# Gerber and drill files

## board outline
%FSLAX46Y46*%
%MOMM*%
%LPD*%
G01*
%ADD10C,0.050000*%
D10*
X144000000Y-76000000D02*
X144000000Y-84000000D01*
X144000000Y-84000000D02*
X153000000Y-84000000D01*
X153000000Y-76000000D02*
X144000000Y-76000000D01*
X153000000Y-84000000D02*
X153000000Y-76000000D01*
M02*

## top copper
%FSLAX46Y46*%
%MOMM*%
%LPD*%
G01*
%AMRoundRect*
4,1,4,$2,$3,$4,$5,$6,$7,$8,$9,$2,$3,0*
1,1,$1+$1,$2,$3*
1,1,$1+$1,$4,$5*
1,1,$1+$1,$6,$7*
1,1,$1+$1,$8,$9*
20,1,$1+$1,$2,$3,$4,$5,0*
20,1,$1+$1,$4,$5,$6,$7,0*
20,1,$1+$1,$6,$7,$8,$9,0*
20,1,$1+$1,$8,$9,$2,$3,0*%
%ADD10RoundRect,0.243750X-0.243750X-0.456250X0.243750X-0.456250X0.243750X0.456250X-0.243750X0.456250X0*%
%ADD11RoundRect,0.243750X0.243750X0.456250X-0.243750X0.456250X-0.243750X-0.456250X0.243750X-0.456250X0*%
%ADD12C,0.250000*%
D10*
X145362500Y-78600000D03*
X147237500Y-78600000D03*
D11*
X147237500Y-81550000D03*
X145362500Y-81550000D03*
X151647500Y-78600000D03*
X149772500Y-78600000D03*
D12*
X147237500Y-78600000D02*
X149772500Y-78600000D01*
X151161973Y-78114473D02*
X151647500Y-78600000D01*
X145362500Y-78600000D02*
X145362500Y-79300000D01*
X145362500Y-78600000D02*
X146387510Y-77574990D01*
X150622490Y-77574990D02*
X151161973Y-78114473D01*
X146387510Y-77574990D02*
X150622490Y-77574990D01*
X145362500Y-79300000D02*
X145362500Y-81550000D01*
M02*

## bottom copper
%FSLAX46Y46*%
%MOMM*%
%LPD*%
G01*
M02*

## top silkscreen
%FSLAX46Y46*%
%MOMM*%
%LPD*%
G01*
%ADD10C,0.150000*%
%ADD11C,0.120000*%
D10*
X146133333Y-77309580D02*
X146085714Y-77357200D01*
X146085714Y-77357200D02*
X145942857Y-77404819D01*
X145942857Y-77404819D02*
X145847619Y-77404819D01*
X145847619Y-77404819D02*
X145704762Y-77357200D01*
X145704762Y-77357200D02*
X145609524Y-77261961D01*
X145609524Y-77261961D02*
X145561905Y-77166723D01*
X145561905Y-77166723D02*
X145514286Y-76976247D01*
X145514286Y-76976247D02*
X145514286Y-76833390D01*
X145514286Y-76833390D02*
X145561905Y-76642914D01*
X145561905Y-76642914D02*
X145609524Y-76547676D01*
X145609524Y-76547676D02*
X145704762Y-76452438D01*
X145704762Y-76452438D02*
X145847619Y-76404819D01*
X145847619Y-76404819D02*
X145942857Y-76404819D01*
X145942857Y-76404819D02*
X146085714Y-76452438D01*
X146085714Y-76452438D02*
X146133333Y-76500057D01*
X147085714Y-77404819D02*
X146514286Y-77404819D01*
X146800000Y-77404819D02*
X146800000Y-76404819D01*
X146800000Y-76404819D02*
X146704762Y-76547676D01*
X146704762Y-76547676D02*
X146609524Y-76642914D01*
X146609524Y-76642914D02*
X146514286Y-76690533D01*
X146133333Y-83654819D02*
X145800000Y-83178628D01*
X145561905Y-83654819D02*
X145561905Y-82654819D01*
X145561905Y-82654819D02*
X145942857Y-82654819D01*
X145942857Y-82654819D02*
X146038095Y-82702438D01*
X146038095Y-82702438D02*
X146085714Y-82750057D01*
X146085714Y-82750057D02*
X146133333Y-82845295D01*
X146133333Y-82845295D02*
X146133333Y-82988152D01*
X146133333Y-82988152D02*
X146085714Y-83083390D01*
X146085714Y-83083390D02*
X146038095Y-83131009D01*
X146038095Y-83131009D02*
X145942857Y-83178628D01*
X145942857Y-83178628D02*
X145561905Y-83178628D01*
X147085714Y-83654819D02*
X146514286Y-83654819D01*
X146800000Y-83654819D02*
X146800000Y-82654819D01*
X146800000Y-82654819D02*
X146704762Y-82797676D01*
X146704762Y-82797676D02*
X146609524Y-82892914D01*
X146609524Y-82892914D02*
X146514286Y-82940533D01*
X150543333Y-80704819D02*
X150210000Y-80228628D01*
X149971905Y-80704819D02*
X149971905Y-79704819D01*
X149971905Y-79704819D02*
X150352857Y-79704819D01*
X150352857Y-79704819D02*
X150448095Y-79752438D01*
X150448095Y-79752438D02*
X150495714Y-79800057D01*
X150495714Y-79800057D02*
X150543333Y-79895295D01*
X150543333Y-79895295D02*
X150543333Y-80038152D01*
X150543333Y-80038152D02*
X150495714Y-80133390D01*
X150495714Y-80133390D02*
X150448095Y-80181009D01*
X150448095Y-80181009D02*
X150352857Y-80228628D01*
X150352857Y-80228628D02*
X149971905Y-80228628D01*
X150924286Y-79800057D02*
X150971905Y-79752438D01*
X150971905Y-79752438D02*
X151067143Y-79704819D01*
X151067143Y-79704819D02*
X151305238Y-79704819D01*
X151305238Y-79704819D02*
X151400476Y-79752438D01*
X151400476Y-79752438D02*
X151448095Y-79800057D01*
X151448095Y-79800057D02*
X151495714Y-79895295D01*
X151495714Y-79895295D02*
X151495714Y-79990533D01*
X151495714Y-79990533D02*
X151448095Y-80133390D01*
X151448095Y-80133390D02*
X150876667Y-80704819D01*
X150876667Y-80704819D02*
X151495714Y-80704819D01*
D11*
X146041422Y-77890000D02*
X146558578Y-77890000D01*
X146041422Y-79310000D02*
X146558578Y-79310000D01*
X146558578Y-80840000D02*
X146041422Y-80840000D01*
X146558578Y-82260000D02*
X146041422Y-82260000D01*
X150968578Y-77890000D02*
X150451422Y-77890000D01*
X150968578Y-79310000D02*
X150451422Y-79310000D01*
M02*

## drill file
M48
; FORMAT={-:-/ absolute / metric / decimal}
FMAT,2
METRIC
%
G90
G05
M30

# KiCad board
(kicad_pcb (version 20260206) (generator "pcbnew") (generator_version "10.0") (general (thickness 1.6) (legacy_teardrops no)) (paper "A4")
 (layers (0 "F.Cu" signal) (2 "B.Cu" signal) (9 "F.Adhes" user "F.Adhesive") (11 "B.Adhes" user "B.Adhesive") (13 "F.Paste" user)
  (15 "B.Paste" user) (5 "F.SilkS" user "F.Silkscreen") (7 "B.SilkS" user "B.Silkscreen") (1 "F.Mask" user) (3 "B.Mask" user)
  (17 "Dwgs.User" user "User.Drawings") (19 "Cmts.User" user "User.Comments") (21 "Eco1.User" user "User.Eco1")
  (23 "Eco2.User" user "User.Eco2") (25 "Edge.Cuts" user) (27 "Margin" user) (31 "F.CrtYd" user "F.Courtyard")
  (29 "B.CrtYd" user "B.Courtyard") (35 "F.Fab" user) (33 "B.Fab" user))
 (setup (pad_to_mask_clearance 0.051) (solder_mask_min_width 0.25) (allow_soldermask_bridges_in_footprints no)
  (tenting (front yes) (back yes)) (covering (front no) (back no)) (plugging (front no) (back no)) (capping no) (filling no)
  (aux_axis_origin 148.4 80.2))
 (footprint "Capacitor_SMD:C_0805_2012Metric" (layer "F.Cu") (at 146.3 78.6)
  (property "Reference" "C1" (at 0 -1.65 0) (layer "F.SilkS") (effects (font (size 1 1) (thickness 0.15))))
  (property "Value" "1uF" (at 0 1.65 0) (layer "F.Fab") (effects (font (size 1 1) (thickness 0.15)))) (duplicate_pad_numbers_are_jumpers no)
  (fp_line (start -0.258578 -0.71) (end 0.258578 -0.71) (stroke (width 0.12) (type solid)) (layer "F.SilkS"))
  (fp_line (start -0.258578 0.71) (end 0.258578 0.71) (stroke (width 0.12) (type solid)) (layer "F.SilkS"))
  (pad "1" smd roundrect (at -0.9375 0) (size 0.975 1.4) (layers "F.Cu" "F.Mask" "F.Paste") (roundrect_rratio 0.25) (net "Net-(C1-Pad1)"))
  (pad "2" smd roundrect (at 0.9375 0) (size 0.975 1.4) (layers "F.Cu" "F.Mask" "F.Paste") (roundrect_rratio 0.25) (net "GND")))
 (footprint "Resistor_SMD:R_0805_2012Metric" (layer "F.Cu") (at 146.3 81.55 180)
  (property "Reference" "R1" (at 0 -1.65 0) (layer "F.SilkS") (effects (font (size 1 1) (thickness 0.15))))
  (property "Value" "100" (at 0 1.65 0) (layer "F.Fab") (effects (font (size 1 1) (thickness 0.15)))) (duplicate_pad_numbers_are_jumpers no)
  (fp_line (start -0.258578 0.71) (end 0.258578 0.71) (stroke (width 0.12) (type solid)) (layer "F.SilkS"))
  (fp_line (start -0.258578 -0.71) (end 0.258578 -0.71) (stroke (width 0.12) (type solid)) (layer "F.SilkS"))
  (pad "1" smd roundrect (at -0.9375 0 180) (size 0.975 1.4) (layers "F.Cu" "F.Mask" "F.Paste") (roundrect_rratio 0.25) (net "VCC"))
  (pad "2" smd roundrect (at 0.9375 0 180) (size 0.975 1.4) (layers "F.Cu" "F.Mask" "F.Paste") (roundrect_rratio 0.25) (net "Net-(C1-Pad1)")))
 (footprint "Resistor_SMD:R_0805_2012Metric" (layer "F.Cu") (at 150.71 78.6 180)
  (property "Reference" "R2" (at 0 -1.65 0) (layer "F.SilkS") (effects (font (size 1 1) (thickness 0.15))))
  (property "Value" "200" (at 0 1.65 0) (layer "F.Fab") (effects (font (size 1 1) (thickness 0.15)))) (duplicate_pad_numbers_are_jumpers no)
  (fp_line (start -0.258578 0.71) (end 0.258578 0.71) (stroke (width 0.12) (type solid)) (layer "F.SilkS"))
  (fp_line (start -0.258578 -0.71) (end 0.258578 -0.71) (stroke (width 0.12) (type solid)) (layer "F.SilkS"))
  (pad "1" smd roundrect (at -0.9375 0 180) (size 0.975 1.4) (layers "F.Cu" "F.Mask" "F.Paste") (roundrect_rratio 0.25)
   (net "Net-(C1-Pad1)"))
  (pad "2" smd roundrect (at 0.9375 0 180) (size 0.975 1.4) (layers "F.Cu" "F.Mask" "F.Paste") (roundrect_rratio 0.25) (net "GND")))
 (gr_line (start 144 76) (end 144 84) (stroke (width 0.05) (type solid)) (layer "Edge.Cuts"))
 (gr_line (start 144 84) (end 153 84) (stroke (width 0.05) (type solid)) (layer "Edge.Cuts"))
 (gr_line (start 153 76) (end 144 76) (stroke (width 0.05) (type solid)) (layer "Edge.Cuts"))
 (gr_line (start 153 84) (end 153 76) (stroke (width 0.05) (type solid)) (layer "Edge.Cuts"))
 (segment (start 147.2375 78.6) (end 149.7725 78.6) (width 0.25) (layer "F.Cu") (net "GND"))
 (segment (start 151.161973 78.114473) (end 151.6475 78.6) (width 0.25) (layer "F.Cu") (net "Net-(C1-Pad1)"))
 (segment (start 145.3625 78.6) (end 145.3625 79.3) (width 0.25) (layer "F.Cu") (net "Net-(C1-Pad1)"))
 (segment (start 145.3625 78.6) (end 146.38751 77.57499) (width 0.25) (layer "F.Cu") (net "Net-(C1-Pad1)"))
 (segment (start 150.62249 77.57499) (end 151.161973 78.114473) (width 0.25) (layer "F.Cu") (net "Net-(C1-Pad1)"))
 (segment (start 146.38751 77.57499) (end 150.62249 77.57499) (width 0.25) (layer "F.Cu") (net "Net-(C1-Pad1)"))
 (segment (start 145.3625 79.3) (end 145.3625 81.55) (width 0.25) (layer "F.Cu") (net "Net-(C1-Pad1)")))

